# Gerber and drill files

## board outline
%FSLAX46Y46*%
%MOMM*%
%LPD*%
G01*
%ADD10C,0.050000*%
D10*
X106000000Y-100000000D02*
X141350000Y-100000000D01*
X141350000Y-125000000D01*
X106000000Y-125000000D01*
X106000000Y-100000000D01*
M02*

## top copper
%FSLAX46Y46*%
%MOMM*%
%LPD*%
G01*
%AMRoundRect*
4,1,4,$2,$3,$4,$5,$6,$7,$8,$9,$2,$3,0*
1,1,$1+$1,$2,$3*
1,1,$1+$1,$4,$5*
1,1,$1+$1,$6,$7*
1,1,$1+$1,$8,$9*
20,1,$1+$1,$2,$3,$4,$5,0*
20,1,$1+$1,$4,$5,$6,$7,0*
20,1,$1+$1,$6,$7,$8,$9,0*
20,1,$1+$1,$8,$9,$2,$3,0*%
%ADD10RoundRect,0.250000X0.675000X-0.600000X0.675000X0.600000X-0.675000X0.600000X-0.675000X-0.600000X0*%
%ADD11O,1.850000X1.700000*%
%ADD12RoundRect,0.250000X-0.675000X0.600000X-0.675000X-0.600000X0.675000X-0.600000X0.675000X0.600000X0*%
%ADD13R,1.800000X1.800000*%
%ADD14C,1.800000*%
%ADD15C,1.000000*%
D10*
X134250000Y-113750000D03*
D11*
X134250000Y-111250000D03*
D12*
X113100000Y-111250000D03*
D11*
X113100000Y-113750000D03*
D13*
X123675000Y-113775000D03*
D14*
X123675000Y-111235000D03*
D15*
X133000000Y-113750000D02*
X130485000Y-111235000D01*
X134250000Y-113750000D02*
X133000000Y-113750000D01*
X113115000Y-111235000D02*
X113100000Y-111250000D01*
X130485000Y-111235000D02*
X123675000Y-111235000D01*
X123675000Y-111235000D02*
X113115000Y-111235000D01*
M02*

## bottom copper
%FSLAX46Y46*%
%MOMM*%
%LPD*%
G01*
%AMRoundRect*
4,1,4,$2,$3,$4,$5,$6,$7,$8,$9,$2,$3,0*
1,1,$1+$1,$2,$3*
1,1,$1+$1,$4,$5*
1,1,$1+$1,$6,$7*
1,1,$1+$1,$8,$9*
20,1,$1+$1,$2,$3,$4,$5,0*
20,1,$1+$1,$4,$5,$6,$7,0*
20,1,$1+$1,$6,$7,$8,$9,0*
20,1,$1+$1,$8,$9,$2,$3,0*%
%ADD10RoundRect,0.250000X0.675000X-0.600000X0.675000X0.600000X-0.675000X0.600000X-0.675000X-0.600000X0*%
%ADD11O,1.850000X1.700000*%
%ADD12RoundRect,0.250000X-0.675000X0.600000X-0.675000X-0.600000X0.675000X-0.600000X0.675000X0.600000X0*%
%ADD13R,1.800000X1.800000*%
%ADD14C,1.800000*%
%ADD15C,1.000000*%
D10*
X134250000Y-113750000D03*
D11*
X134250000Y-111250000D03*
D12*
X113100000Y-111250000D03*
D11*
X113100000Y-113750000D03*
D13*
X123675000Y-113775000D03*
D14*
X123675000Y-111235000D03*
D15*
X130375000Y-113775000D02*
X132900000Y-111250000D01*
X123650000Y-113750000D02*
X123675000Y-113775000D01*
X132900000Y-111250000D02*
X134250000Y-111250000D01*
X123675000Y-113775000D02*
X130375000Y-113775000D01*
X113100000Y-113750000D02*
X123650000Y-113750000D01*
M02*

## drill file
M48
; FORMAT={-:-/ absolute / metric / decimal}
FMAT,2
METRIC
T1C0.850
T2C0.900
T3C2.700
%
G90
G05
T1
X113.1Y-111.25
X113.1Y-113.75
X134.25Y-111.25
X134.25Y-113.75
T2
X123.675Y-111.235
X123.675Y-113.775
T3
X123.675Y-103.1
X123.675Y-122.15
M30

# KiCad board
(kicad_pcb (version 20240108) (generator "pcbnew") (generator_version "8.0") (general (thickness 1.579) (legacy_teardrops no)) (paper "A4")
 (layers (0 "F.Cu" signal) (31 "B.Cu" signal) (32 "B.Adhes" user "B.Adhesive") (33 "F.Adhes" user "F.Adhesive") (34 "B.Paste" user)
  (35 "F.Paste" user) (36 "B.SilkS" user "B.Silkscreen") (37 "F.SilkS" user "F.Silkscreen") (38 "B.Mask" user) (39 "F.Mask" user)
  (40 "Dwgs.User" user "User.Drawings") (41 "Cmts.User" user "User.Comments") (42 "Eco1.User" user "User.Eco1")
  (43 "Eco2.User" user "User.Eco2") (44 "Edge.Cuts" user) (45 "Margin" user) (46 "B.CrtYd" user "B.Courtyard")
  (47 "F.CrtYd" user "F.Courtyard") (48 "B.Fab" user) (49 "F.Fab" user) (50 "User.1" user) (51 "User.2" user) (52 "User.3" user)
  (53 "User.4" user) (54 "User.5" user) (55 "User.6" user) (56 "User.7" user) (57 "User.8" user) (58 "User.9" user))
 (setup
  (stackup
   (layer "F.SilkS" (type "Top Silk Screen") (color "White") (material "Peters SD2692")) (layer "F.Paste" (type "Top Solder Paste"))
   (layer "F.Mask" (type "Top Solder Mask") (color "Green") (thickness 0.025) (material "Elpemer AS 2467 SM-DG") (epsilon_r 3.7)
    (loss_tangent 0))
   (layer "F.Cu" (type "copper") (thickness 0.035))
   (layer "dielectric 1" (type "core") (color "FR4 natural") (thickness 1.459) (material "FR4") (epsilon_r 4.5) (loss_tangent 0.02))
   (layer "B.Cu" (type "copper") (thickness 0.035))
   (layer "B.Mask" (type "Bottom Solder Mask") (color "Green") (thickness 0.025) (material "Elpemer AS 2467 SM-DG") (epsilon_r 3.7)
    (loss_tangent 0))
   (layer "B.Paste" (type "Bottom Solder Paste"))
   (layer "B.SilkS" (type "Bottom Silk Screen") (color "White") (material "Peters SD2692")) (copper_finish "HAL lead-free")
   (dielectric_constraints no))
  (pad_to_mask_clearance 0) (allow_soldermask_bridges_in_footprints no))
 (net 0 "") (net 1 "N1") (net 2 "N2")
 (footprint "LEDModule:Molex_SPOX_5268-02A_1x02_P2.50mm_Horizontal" (layer "F.Cu") (at 134.25 113.75 90)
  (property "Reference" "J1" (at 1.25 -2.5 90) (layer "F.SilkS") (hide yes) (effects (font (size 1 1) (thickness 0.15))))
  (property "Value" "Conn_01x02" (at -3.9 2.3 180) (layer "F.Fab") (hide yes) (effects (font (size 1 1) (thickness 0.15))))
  (pad "1" thru_hole roundrect (at 0 0 90) (size 1.7 1.85) (drill 0.85) (layers "*.Cu" "*.Mask") (remove_unused_layers no)
   (roundrect_rratio 0.147059) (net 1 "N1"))
  (pad "2" thru_hole oval (at 2.5 0 90) (size 1.7 1.85) (drill 0.85) (layers "*.Cu" "*.Mask") (remove_unused_layers no) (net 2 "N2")))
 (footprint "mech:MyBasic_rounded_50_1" (layer "F.Cu") (at 109.6 102.6)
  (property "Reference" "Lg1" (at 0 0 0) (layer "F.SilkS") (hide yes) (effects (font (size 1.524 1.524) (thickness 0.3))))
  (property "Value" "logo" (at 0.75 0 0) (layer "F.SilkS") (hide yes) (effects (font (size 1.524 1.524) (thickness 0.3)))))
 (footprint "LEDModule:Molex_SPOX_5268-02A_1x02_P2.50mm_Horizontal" (layer "F.Cu") (at 113.1 111.25 -90)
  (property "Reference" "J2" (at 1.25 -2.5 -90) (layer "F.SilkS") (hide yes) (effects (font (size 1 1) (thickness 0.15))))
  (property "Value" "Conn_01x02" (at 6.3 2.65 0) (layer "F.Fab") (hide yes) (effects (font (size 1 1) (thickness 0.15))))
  (pad "1" thru_hole roundrect (at 0 0 270) (size 1.7 1.85) (drill 0.85) (layers "*.Cu" "*.Mask") (remove_unused_layers no)
   (roundrect_rratio 0.147059) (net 1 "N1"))
  (pad "2" thru_hole oval (at 2.5 0 270) (size 1.7 1.85) (drill 0.85) (layers "*.Cu" "*.Mask") (remove_unused_layers no) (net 2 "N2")))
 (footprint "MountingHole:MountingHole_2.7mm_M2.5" (layer "F.Cu") (at 123.675 122.15)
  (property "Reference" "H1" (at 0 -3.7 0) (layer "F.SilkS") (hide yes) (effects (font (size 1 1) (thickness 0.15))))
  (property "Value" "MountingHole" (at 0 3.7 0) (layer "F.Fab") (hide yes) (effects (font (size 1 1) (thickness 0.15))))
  (pad "" np_thru_hole circle (at 0 0) (size 2.7 2.7) (drill 2.7) (layers "*.Cu" "*.Mask")))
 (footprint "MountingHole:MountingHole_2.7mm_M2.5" (layer "F.Cu") (at 123.675 103.1)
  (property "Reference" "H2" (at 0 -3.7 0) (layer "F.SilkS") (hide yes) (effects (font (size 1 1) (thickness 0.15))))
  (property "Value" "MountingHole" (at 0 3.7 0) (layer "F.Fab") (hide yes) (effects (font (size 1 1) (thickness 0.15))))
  (pad "" np_thru_hole circle (at 0 0) (size 2.7 2.7) (drill 2.7) (layers "*.Cu" "*.Mask")))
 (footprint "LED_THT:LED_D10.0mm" (layer "F.Cu") (at 123.675 113.775 90)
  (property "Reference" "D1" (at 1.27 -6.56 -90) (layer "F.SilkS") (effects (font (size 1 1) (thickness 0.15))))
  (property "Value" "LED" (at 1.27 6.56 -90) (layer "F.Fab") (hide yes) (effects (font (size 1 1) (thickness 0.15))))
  (pad "1" thru_hole rect (at 0 0 90) (size 1.8 1.8) (drill 0.9) (layers "*.Cu" "*.Mask") (remove_unused_layers no) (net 2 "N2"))
  (pad "2" thru_hole circle (at 2.54 0 90) (size 1.8 1.8) (drill 0.9) (layers "*.Cu" "*.Mask") (remove_unused_layers no) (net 1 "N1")))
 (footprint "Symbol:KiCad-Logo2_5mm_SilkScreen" (layer "B.Cu") (at 112.75 121.7 180)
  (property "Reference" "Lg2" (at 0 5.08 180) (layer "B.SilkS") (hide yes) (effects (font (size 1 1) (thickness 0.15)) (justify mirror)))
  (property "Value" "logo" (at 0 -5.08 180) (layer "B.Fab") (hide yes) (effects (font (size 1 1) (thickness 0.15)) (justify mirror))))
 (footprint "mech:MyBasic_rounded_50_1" (layer "B.Cu") (at 137.8 102.6 180)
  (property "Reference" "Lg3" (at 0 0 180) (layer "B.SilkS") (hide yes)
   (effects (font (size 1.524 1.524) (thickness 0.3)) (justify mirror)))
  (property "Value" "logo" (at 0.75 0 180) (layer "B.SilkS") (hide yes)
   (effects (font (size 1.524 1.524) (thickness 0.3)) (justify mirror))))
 (gr_rect (start 106 100) (end 141.35 125) (stroke (width 0.05) (type default)) (fill none) (layer "Edge.Cuts"))
 (segment (start 130.375 113.775) (end 132.9 111.25) (width 1) (layer "B.Cu") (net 2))
 (segment (start 123.65 113.75) (end 123.675 113.775) (width 1) (layer "B.Cu") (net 2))
 (segment (start 132.9 111.25) (end 134.25 111.25) (width 1) (layer "B.Cu") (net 2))
 (segment (start 123.675 113.775) (end 130.375 113.775) (width 1) (layer "B.Cu") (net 2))
 (segment (start 113.1 113.75) (end 123.65 113.75) (width 1) (layer "B.Cu") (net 2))
 (segment (start 133 113.75) (end 130.485 111.235) (width 1) (layer "F.Cu") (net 1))
 (segment (start 134.25 113.75) (end 133 113.75) (width 1) (layer "F.Cu") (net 1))
 (segment (start 113.115 111.235) (end 113.1 111.25) (width 1) (layer "F.Cu") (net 1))
 (segment (start 130.485 111.235) (end 123.675 111.235) (width 1) (layer "F.Cu") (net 1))
 (segment (start 123.675 111.235) (end 113.115 111.235) (width 1) (layer "F.Cu") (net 1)))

